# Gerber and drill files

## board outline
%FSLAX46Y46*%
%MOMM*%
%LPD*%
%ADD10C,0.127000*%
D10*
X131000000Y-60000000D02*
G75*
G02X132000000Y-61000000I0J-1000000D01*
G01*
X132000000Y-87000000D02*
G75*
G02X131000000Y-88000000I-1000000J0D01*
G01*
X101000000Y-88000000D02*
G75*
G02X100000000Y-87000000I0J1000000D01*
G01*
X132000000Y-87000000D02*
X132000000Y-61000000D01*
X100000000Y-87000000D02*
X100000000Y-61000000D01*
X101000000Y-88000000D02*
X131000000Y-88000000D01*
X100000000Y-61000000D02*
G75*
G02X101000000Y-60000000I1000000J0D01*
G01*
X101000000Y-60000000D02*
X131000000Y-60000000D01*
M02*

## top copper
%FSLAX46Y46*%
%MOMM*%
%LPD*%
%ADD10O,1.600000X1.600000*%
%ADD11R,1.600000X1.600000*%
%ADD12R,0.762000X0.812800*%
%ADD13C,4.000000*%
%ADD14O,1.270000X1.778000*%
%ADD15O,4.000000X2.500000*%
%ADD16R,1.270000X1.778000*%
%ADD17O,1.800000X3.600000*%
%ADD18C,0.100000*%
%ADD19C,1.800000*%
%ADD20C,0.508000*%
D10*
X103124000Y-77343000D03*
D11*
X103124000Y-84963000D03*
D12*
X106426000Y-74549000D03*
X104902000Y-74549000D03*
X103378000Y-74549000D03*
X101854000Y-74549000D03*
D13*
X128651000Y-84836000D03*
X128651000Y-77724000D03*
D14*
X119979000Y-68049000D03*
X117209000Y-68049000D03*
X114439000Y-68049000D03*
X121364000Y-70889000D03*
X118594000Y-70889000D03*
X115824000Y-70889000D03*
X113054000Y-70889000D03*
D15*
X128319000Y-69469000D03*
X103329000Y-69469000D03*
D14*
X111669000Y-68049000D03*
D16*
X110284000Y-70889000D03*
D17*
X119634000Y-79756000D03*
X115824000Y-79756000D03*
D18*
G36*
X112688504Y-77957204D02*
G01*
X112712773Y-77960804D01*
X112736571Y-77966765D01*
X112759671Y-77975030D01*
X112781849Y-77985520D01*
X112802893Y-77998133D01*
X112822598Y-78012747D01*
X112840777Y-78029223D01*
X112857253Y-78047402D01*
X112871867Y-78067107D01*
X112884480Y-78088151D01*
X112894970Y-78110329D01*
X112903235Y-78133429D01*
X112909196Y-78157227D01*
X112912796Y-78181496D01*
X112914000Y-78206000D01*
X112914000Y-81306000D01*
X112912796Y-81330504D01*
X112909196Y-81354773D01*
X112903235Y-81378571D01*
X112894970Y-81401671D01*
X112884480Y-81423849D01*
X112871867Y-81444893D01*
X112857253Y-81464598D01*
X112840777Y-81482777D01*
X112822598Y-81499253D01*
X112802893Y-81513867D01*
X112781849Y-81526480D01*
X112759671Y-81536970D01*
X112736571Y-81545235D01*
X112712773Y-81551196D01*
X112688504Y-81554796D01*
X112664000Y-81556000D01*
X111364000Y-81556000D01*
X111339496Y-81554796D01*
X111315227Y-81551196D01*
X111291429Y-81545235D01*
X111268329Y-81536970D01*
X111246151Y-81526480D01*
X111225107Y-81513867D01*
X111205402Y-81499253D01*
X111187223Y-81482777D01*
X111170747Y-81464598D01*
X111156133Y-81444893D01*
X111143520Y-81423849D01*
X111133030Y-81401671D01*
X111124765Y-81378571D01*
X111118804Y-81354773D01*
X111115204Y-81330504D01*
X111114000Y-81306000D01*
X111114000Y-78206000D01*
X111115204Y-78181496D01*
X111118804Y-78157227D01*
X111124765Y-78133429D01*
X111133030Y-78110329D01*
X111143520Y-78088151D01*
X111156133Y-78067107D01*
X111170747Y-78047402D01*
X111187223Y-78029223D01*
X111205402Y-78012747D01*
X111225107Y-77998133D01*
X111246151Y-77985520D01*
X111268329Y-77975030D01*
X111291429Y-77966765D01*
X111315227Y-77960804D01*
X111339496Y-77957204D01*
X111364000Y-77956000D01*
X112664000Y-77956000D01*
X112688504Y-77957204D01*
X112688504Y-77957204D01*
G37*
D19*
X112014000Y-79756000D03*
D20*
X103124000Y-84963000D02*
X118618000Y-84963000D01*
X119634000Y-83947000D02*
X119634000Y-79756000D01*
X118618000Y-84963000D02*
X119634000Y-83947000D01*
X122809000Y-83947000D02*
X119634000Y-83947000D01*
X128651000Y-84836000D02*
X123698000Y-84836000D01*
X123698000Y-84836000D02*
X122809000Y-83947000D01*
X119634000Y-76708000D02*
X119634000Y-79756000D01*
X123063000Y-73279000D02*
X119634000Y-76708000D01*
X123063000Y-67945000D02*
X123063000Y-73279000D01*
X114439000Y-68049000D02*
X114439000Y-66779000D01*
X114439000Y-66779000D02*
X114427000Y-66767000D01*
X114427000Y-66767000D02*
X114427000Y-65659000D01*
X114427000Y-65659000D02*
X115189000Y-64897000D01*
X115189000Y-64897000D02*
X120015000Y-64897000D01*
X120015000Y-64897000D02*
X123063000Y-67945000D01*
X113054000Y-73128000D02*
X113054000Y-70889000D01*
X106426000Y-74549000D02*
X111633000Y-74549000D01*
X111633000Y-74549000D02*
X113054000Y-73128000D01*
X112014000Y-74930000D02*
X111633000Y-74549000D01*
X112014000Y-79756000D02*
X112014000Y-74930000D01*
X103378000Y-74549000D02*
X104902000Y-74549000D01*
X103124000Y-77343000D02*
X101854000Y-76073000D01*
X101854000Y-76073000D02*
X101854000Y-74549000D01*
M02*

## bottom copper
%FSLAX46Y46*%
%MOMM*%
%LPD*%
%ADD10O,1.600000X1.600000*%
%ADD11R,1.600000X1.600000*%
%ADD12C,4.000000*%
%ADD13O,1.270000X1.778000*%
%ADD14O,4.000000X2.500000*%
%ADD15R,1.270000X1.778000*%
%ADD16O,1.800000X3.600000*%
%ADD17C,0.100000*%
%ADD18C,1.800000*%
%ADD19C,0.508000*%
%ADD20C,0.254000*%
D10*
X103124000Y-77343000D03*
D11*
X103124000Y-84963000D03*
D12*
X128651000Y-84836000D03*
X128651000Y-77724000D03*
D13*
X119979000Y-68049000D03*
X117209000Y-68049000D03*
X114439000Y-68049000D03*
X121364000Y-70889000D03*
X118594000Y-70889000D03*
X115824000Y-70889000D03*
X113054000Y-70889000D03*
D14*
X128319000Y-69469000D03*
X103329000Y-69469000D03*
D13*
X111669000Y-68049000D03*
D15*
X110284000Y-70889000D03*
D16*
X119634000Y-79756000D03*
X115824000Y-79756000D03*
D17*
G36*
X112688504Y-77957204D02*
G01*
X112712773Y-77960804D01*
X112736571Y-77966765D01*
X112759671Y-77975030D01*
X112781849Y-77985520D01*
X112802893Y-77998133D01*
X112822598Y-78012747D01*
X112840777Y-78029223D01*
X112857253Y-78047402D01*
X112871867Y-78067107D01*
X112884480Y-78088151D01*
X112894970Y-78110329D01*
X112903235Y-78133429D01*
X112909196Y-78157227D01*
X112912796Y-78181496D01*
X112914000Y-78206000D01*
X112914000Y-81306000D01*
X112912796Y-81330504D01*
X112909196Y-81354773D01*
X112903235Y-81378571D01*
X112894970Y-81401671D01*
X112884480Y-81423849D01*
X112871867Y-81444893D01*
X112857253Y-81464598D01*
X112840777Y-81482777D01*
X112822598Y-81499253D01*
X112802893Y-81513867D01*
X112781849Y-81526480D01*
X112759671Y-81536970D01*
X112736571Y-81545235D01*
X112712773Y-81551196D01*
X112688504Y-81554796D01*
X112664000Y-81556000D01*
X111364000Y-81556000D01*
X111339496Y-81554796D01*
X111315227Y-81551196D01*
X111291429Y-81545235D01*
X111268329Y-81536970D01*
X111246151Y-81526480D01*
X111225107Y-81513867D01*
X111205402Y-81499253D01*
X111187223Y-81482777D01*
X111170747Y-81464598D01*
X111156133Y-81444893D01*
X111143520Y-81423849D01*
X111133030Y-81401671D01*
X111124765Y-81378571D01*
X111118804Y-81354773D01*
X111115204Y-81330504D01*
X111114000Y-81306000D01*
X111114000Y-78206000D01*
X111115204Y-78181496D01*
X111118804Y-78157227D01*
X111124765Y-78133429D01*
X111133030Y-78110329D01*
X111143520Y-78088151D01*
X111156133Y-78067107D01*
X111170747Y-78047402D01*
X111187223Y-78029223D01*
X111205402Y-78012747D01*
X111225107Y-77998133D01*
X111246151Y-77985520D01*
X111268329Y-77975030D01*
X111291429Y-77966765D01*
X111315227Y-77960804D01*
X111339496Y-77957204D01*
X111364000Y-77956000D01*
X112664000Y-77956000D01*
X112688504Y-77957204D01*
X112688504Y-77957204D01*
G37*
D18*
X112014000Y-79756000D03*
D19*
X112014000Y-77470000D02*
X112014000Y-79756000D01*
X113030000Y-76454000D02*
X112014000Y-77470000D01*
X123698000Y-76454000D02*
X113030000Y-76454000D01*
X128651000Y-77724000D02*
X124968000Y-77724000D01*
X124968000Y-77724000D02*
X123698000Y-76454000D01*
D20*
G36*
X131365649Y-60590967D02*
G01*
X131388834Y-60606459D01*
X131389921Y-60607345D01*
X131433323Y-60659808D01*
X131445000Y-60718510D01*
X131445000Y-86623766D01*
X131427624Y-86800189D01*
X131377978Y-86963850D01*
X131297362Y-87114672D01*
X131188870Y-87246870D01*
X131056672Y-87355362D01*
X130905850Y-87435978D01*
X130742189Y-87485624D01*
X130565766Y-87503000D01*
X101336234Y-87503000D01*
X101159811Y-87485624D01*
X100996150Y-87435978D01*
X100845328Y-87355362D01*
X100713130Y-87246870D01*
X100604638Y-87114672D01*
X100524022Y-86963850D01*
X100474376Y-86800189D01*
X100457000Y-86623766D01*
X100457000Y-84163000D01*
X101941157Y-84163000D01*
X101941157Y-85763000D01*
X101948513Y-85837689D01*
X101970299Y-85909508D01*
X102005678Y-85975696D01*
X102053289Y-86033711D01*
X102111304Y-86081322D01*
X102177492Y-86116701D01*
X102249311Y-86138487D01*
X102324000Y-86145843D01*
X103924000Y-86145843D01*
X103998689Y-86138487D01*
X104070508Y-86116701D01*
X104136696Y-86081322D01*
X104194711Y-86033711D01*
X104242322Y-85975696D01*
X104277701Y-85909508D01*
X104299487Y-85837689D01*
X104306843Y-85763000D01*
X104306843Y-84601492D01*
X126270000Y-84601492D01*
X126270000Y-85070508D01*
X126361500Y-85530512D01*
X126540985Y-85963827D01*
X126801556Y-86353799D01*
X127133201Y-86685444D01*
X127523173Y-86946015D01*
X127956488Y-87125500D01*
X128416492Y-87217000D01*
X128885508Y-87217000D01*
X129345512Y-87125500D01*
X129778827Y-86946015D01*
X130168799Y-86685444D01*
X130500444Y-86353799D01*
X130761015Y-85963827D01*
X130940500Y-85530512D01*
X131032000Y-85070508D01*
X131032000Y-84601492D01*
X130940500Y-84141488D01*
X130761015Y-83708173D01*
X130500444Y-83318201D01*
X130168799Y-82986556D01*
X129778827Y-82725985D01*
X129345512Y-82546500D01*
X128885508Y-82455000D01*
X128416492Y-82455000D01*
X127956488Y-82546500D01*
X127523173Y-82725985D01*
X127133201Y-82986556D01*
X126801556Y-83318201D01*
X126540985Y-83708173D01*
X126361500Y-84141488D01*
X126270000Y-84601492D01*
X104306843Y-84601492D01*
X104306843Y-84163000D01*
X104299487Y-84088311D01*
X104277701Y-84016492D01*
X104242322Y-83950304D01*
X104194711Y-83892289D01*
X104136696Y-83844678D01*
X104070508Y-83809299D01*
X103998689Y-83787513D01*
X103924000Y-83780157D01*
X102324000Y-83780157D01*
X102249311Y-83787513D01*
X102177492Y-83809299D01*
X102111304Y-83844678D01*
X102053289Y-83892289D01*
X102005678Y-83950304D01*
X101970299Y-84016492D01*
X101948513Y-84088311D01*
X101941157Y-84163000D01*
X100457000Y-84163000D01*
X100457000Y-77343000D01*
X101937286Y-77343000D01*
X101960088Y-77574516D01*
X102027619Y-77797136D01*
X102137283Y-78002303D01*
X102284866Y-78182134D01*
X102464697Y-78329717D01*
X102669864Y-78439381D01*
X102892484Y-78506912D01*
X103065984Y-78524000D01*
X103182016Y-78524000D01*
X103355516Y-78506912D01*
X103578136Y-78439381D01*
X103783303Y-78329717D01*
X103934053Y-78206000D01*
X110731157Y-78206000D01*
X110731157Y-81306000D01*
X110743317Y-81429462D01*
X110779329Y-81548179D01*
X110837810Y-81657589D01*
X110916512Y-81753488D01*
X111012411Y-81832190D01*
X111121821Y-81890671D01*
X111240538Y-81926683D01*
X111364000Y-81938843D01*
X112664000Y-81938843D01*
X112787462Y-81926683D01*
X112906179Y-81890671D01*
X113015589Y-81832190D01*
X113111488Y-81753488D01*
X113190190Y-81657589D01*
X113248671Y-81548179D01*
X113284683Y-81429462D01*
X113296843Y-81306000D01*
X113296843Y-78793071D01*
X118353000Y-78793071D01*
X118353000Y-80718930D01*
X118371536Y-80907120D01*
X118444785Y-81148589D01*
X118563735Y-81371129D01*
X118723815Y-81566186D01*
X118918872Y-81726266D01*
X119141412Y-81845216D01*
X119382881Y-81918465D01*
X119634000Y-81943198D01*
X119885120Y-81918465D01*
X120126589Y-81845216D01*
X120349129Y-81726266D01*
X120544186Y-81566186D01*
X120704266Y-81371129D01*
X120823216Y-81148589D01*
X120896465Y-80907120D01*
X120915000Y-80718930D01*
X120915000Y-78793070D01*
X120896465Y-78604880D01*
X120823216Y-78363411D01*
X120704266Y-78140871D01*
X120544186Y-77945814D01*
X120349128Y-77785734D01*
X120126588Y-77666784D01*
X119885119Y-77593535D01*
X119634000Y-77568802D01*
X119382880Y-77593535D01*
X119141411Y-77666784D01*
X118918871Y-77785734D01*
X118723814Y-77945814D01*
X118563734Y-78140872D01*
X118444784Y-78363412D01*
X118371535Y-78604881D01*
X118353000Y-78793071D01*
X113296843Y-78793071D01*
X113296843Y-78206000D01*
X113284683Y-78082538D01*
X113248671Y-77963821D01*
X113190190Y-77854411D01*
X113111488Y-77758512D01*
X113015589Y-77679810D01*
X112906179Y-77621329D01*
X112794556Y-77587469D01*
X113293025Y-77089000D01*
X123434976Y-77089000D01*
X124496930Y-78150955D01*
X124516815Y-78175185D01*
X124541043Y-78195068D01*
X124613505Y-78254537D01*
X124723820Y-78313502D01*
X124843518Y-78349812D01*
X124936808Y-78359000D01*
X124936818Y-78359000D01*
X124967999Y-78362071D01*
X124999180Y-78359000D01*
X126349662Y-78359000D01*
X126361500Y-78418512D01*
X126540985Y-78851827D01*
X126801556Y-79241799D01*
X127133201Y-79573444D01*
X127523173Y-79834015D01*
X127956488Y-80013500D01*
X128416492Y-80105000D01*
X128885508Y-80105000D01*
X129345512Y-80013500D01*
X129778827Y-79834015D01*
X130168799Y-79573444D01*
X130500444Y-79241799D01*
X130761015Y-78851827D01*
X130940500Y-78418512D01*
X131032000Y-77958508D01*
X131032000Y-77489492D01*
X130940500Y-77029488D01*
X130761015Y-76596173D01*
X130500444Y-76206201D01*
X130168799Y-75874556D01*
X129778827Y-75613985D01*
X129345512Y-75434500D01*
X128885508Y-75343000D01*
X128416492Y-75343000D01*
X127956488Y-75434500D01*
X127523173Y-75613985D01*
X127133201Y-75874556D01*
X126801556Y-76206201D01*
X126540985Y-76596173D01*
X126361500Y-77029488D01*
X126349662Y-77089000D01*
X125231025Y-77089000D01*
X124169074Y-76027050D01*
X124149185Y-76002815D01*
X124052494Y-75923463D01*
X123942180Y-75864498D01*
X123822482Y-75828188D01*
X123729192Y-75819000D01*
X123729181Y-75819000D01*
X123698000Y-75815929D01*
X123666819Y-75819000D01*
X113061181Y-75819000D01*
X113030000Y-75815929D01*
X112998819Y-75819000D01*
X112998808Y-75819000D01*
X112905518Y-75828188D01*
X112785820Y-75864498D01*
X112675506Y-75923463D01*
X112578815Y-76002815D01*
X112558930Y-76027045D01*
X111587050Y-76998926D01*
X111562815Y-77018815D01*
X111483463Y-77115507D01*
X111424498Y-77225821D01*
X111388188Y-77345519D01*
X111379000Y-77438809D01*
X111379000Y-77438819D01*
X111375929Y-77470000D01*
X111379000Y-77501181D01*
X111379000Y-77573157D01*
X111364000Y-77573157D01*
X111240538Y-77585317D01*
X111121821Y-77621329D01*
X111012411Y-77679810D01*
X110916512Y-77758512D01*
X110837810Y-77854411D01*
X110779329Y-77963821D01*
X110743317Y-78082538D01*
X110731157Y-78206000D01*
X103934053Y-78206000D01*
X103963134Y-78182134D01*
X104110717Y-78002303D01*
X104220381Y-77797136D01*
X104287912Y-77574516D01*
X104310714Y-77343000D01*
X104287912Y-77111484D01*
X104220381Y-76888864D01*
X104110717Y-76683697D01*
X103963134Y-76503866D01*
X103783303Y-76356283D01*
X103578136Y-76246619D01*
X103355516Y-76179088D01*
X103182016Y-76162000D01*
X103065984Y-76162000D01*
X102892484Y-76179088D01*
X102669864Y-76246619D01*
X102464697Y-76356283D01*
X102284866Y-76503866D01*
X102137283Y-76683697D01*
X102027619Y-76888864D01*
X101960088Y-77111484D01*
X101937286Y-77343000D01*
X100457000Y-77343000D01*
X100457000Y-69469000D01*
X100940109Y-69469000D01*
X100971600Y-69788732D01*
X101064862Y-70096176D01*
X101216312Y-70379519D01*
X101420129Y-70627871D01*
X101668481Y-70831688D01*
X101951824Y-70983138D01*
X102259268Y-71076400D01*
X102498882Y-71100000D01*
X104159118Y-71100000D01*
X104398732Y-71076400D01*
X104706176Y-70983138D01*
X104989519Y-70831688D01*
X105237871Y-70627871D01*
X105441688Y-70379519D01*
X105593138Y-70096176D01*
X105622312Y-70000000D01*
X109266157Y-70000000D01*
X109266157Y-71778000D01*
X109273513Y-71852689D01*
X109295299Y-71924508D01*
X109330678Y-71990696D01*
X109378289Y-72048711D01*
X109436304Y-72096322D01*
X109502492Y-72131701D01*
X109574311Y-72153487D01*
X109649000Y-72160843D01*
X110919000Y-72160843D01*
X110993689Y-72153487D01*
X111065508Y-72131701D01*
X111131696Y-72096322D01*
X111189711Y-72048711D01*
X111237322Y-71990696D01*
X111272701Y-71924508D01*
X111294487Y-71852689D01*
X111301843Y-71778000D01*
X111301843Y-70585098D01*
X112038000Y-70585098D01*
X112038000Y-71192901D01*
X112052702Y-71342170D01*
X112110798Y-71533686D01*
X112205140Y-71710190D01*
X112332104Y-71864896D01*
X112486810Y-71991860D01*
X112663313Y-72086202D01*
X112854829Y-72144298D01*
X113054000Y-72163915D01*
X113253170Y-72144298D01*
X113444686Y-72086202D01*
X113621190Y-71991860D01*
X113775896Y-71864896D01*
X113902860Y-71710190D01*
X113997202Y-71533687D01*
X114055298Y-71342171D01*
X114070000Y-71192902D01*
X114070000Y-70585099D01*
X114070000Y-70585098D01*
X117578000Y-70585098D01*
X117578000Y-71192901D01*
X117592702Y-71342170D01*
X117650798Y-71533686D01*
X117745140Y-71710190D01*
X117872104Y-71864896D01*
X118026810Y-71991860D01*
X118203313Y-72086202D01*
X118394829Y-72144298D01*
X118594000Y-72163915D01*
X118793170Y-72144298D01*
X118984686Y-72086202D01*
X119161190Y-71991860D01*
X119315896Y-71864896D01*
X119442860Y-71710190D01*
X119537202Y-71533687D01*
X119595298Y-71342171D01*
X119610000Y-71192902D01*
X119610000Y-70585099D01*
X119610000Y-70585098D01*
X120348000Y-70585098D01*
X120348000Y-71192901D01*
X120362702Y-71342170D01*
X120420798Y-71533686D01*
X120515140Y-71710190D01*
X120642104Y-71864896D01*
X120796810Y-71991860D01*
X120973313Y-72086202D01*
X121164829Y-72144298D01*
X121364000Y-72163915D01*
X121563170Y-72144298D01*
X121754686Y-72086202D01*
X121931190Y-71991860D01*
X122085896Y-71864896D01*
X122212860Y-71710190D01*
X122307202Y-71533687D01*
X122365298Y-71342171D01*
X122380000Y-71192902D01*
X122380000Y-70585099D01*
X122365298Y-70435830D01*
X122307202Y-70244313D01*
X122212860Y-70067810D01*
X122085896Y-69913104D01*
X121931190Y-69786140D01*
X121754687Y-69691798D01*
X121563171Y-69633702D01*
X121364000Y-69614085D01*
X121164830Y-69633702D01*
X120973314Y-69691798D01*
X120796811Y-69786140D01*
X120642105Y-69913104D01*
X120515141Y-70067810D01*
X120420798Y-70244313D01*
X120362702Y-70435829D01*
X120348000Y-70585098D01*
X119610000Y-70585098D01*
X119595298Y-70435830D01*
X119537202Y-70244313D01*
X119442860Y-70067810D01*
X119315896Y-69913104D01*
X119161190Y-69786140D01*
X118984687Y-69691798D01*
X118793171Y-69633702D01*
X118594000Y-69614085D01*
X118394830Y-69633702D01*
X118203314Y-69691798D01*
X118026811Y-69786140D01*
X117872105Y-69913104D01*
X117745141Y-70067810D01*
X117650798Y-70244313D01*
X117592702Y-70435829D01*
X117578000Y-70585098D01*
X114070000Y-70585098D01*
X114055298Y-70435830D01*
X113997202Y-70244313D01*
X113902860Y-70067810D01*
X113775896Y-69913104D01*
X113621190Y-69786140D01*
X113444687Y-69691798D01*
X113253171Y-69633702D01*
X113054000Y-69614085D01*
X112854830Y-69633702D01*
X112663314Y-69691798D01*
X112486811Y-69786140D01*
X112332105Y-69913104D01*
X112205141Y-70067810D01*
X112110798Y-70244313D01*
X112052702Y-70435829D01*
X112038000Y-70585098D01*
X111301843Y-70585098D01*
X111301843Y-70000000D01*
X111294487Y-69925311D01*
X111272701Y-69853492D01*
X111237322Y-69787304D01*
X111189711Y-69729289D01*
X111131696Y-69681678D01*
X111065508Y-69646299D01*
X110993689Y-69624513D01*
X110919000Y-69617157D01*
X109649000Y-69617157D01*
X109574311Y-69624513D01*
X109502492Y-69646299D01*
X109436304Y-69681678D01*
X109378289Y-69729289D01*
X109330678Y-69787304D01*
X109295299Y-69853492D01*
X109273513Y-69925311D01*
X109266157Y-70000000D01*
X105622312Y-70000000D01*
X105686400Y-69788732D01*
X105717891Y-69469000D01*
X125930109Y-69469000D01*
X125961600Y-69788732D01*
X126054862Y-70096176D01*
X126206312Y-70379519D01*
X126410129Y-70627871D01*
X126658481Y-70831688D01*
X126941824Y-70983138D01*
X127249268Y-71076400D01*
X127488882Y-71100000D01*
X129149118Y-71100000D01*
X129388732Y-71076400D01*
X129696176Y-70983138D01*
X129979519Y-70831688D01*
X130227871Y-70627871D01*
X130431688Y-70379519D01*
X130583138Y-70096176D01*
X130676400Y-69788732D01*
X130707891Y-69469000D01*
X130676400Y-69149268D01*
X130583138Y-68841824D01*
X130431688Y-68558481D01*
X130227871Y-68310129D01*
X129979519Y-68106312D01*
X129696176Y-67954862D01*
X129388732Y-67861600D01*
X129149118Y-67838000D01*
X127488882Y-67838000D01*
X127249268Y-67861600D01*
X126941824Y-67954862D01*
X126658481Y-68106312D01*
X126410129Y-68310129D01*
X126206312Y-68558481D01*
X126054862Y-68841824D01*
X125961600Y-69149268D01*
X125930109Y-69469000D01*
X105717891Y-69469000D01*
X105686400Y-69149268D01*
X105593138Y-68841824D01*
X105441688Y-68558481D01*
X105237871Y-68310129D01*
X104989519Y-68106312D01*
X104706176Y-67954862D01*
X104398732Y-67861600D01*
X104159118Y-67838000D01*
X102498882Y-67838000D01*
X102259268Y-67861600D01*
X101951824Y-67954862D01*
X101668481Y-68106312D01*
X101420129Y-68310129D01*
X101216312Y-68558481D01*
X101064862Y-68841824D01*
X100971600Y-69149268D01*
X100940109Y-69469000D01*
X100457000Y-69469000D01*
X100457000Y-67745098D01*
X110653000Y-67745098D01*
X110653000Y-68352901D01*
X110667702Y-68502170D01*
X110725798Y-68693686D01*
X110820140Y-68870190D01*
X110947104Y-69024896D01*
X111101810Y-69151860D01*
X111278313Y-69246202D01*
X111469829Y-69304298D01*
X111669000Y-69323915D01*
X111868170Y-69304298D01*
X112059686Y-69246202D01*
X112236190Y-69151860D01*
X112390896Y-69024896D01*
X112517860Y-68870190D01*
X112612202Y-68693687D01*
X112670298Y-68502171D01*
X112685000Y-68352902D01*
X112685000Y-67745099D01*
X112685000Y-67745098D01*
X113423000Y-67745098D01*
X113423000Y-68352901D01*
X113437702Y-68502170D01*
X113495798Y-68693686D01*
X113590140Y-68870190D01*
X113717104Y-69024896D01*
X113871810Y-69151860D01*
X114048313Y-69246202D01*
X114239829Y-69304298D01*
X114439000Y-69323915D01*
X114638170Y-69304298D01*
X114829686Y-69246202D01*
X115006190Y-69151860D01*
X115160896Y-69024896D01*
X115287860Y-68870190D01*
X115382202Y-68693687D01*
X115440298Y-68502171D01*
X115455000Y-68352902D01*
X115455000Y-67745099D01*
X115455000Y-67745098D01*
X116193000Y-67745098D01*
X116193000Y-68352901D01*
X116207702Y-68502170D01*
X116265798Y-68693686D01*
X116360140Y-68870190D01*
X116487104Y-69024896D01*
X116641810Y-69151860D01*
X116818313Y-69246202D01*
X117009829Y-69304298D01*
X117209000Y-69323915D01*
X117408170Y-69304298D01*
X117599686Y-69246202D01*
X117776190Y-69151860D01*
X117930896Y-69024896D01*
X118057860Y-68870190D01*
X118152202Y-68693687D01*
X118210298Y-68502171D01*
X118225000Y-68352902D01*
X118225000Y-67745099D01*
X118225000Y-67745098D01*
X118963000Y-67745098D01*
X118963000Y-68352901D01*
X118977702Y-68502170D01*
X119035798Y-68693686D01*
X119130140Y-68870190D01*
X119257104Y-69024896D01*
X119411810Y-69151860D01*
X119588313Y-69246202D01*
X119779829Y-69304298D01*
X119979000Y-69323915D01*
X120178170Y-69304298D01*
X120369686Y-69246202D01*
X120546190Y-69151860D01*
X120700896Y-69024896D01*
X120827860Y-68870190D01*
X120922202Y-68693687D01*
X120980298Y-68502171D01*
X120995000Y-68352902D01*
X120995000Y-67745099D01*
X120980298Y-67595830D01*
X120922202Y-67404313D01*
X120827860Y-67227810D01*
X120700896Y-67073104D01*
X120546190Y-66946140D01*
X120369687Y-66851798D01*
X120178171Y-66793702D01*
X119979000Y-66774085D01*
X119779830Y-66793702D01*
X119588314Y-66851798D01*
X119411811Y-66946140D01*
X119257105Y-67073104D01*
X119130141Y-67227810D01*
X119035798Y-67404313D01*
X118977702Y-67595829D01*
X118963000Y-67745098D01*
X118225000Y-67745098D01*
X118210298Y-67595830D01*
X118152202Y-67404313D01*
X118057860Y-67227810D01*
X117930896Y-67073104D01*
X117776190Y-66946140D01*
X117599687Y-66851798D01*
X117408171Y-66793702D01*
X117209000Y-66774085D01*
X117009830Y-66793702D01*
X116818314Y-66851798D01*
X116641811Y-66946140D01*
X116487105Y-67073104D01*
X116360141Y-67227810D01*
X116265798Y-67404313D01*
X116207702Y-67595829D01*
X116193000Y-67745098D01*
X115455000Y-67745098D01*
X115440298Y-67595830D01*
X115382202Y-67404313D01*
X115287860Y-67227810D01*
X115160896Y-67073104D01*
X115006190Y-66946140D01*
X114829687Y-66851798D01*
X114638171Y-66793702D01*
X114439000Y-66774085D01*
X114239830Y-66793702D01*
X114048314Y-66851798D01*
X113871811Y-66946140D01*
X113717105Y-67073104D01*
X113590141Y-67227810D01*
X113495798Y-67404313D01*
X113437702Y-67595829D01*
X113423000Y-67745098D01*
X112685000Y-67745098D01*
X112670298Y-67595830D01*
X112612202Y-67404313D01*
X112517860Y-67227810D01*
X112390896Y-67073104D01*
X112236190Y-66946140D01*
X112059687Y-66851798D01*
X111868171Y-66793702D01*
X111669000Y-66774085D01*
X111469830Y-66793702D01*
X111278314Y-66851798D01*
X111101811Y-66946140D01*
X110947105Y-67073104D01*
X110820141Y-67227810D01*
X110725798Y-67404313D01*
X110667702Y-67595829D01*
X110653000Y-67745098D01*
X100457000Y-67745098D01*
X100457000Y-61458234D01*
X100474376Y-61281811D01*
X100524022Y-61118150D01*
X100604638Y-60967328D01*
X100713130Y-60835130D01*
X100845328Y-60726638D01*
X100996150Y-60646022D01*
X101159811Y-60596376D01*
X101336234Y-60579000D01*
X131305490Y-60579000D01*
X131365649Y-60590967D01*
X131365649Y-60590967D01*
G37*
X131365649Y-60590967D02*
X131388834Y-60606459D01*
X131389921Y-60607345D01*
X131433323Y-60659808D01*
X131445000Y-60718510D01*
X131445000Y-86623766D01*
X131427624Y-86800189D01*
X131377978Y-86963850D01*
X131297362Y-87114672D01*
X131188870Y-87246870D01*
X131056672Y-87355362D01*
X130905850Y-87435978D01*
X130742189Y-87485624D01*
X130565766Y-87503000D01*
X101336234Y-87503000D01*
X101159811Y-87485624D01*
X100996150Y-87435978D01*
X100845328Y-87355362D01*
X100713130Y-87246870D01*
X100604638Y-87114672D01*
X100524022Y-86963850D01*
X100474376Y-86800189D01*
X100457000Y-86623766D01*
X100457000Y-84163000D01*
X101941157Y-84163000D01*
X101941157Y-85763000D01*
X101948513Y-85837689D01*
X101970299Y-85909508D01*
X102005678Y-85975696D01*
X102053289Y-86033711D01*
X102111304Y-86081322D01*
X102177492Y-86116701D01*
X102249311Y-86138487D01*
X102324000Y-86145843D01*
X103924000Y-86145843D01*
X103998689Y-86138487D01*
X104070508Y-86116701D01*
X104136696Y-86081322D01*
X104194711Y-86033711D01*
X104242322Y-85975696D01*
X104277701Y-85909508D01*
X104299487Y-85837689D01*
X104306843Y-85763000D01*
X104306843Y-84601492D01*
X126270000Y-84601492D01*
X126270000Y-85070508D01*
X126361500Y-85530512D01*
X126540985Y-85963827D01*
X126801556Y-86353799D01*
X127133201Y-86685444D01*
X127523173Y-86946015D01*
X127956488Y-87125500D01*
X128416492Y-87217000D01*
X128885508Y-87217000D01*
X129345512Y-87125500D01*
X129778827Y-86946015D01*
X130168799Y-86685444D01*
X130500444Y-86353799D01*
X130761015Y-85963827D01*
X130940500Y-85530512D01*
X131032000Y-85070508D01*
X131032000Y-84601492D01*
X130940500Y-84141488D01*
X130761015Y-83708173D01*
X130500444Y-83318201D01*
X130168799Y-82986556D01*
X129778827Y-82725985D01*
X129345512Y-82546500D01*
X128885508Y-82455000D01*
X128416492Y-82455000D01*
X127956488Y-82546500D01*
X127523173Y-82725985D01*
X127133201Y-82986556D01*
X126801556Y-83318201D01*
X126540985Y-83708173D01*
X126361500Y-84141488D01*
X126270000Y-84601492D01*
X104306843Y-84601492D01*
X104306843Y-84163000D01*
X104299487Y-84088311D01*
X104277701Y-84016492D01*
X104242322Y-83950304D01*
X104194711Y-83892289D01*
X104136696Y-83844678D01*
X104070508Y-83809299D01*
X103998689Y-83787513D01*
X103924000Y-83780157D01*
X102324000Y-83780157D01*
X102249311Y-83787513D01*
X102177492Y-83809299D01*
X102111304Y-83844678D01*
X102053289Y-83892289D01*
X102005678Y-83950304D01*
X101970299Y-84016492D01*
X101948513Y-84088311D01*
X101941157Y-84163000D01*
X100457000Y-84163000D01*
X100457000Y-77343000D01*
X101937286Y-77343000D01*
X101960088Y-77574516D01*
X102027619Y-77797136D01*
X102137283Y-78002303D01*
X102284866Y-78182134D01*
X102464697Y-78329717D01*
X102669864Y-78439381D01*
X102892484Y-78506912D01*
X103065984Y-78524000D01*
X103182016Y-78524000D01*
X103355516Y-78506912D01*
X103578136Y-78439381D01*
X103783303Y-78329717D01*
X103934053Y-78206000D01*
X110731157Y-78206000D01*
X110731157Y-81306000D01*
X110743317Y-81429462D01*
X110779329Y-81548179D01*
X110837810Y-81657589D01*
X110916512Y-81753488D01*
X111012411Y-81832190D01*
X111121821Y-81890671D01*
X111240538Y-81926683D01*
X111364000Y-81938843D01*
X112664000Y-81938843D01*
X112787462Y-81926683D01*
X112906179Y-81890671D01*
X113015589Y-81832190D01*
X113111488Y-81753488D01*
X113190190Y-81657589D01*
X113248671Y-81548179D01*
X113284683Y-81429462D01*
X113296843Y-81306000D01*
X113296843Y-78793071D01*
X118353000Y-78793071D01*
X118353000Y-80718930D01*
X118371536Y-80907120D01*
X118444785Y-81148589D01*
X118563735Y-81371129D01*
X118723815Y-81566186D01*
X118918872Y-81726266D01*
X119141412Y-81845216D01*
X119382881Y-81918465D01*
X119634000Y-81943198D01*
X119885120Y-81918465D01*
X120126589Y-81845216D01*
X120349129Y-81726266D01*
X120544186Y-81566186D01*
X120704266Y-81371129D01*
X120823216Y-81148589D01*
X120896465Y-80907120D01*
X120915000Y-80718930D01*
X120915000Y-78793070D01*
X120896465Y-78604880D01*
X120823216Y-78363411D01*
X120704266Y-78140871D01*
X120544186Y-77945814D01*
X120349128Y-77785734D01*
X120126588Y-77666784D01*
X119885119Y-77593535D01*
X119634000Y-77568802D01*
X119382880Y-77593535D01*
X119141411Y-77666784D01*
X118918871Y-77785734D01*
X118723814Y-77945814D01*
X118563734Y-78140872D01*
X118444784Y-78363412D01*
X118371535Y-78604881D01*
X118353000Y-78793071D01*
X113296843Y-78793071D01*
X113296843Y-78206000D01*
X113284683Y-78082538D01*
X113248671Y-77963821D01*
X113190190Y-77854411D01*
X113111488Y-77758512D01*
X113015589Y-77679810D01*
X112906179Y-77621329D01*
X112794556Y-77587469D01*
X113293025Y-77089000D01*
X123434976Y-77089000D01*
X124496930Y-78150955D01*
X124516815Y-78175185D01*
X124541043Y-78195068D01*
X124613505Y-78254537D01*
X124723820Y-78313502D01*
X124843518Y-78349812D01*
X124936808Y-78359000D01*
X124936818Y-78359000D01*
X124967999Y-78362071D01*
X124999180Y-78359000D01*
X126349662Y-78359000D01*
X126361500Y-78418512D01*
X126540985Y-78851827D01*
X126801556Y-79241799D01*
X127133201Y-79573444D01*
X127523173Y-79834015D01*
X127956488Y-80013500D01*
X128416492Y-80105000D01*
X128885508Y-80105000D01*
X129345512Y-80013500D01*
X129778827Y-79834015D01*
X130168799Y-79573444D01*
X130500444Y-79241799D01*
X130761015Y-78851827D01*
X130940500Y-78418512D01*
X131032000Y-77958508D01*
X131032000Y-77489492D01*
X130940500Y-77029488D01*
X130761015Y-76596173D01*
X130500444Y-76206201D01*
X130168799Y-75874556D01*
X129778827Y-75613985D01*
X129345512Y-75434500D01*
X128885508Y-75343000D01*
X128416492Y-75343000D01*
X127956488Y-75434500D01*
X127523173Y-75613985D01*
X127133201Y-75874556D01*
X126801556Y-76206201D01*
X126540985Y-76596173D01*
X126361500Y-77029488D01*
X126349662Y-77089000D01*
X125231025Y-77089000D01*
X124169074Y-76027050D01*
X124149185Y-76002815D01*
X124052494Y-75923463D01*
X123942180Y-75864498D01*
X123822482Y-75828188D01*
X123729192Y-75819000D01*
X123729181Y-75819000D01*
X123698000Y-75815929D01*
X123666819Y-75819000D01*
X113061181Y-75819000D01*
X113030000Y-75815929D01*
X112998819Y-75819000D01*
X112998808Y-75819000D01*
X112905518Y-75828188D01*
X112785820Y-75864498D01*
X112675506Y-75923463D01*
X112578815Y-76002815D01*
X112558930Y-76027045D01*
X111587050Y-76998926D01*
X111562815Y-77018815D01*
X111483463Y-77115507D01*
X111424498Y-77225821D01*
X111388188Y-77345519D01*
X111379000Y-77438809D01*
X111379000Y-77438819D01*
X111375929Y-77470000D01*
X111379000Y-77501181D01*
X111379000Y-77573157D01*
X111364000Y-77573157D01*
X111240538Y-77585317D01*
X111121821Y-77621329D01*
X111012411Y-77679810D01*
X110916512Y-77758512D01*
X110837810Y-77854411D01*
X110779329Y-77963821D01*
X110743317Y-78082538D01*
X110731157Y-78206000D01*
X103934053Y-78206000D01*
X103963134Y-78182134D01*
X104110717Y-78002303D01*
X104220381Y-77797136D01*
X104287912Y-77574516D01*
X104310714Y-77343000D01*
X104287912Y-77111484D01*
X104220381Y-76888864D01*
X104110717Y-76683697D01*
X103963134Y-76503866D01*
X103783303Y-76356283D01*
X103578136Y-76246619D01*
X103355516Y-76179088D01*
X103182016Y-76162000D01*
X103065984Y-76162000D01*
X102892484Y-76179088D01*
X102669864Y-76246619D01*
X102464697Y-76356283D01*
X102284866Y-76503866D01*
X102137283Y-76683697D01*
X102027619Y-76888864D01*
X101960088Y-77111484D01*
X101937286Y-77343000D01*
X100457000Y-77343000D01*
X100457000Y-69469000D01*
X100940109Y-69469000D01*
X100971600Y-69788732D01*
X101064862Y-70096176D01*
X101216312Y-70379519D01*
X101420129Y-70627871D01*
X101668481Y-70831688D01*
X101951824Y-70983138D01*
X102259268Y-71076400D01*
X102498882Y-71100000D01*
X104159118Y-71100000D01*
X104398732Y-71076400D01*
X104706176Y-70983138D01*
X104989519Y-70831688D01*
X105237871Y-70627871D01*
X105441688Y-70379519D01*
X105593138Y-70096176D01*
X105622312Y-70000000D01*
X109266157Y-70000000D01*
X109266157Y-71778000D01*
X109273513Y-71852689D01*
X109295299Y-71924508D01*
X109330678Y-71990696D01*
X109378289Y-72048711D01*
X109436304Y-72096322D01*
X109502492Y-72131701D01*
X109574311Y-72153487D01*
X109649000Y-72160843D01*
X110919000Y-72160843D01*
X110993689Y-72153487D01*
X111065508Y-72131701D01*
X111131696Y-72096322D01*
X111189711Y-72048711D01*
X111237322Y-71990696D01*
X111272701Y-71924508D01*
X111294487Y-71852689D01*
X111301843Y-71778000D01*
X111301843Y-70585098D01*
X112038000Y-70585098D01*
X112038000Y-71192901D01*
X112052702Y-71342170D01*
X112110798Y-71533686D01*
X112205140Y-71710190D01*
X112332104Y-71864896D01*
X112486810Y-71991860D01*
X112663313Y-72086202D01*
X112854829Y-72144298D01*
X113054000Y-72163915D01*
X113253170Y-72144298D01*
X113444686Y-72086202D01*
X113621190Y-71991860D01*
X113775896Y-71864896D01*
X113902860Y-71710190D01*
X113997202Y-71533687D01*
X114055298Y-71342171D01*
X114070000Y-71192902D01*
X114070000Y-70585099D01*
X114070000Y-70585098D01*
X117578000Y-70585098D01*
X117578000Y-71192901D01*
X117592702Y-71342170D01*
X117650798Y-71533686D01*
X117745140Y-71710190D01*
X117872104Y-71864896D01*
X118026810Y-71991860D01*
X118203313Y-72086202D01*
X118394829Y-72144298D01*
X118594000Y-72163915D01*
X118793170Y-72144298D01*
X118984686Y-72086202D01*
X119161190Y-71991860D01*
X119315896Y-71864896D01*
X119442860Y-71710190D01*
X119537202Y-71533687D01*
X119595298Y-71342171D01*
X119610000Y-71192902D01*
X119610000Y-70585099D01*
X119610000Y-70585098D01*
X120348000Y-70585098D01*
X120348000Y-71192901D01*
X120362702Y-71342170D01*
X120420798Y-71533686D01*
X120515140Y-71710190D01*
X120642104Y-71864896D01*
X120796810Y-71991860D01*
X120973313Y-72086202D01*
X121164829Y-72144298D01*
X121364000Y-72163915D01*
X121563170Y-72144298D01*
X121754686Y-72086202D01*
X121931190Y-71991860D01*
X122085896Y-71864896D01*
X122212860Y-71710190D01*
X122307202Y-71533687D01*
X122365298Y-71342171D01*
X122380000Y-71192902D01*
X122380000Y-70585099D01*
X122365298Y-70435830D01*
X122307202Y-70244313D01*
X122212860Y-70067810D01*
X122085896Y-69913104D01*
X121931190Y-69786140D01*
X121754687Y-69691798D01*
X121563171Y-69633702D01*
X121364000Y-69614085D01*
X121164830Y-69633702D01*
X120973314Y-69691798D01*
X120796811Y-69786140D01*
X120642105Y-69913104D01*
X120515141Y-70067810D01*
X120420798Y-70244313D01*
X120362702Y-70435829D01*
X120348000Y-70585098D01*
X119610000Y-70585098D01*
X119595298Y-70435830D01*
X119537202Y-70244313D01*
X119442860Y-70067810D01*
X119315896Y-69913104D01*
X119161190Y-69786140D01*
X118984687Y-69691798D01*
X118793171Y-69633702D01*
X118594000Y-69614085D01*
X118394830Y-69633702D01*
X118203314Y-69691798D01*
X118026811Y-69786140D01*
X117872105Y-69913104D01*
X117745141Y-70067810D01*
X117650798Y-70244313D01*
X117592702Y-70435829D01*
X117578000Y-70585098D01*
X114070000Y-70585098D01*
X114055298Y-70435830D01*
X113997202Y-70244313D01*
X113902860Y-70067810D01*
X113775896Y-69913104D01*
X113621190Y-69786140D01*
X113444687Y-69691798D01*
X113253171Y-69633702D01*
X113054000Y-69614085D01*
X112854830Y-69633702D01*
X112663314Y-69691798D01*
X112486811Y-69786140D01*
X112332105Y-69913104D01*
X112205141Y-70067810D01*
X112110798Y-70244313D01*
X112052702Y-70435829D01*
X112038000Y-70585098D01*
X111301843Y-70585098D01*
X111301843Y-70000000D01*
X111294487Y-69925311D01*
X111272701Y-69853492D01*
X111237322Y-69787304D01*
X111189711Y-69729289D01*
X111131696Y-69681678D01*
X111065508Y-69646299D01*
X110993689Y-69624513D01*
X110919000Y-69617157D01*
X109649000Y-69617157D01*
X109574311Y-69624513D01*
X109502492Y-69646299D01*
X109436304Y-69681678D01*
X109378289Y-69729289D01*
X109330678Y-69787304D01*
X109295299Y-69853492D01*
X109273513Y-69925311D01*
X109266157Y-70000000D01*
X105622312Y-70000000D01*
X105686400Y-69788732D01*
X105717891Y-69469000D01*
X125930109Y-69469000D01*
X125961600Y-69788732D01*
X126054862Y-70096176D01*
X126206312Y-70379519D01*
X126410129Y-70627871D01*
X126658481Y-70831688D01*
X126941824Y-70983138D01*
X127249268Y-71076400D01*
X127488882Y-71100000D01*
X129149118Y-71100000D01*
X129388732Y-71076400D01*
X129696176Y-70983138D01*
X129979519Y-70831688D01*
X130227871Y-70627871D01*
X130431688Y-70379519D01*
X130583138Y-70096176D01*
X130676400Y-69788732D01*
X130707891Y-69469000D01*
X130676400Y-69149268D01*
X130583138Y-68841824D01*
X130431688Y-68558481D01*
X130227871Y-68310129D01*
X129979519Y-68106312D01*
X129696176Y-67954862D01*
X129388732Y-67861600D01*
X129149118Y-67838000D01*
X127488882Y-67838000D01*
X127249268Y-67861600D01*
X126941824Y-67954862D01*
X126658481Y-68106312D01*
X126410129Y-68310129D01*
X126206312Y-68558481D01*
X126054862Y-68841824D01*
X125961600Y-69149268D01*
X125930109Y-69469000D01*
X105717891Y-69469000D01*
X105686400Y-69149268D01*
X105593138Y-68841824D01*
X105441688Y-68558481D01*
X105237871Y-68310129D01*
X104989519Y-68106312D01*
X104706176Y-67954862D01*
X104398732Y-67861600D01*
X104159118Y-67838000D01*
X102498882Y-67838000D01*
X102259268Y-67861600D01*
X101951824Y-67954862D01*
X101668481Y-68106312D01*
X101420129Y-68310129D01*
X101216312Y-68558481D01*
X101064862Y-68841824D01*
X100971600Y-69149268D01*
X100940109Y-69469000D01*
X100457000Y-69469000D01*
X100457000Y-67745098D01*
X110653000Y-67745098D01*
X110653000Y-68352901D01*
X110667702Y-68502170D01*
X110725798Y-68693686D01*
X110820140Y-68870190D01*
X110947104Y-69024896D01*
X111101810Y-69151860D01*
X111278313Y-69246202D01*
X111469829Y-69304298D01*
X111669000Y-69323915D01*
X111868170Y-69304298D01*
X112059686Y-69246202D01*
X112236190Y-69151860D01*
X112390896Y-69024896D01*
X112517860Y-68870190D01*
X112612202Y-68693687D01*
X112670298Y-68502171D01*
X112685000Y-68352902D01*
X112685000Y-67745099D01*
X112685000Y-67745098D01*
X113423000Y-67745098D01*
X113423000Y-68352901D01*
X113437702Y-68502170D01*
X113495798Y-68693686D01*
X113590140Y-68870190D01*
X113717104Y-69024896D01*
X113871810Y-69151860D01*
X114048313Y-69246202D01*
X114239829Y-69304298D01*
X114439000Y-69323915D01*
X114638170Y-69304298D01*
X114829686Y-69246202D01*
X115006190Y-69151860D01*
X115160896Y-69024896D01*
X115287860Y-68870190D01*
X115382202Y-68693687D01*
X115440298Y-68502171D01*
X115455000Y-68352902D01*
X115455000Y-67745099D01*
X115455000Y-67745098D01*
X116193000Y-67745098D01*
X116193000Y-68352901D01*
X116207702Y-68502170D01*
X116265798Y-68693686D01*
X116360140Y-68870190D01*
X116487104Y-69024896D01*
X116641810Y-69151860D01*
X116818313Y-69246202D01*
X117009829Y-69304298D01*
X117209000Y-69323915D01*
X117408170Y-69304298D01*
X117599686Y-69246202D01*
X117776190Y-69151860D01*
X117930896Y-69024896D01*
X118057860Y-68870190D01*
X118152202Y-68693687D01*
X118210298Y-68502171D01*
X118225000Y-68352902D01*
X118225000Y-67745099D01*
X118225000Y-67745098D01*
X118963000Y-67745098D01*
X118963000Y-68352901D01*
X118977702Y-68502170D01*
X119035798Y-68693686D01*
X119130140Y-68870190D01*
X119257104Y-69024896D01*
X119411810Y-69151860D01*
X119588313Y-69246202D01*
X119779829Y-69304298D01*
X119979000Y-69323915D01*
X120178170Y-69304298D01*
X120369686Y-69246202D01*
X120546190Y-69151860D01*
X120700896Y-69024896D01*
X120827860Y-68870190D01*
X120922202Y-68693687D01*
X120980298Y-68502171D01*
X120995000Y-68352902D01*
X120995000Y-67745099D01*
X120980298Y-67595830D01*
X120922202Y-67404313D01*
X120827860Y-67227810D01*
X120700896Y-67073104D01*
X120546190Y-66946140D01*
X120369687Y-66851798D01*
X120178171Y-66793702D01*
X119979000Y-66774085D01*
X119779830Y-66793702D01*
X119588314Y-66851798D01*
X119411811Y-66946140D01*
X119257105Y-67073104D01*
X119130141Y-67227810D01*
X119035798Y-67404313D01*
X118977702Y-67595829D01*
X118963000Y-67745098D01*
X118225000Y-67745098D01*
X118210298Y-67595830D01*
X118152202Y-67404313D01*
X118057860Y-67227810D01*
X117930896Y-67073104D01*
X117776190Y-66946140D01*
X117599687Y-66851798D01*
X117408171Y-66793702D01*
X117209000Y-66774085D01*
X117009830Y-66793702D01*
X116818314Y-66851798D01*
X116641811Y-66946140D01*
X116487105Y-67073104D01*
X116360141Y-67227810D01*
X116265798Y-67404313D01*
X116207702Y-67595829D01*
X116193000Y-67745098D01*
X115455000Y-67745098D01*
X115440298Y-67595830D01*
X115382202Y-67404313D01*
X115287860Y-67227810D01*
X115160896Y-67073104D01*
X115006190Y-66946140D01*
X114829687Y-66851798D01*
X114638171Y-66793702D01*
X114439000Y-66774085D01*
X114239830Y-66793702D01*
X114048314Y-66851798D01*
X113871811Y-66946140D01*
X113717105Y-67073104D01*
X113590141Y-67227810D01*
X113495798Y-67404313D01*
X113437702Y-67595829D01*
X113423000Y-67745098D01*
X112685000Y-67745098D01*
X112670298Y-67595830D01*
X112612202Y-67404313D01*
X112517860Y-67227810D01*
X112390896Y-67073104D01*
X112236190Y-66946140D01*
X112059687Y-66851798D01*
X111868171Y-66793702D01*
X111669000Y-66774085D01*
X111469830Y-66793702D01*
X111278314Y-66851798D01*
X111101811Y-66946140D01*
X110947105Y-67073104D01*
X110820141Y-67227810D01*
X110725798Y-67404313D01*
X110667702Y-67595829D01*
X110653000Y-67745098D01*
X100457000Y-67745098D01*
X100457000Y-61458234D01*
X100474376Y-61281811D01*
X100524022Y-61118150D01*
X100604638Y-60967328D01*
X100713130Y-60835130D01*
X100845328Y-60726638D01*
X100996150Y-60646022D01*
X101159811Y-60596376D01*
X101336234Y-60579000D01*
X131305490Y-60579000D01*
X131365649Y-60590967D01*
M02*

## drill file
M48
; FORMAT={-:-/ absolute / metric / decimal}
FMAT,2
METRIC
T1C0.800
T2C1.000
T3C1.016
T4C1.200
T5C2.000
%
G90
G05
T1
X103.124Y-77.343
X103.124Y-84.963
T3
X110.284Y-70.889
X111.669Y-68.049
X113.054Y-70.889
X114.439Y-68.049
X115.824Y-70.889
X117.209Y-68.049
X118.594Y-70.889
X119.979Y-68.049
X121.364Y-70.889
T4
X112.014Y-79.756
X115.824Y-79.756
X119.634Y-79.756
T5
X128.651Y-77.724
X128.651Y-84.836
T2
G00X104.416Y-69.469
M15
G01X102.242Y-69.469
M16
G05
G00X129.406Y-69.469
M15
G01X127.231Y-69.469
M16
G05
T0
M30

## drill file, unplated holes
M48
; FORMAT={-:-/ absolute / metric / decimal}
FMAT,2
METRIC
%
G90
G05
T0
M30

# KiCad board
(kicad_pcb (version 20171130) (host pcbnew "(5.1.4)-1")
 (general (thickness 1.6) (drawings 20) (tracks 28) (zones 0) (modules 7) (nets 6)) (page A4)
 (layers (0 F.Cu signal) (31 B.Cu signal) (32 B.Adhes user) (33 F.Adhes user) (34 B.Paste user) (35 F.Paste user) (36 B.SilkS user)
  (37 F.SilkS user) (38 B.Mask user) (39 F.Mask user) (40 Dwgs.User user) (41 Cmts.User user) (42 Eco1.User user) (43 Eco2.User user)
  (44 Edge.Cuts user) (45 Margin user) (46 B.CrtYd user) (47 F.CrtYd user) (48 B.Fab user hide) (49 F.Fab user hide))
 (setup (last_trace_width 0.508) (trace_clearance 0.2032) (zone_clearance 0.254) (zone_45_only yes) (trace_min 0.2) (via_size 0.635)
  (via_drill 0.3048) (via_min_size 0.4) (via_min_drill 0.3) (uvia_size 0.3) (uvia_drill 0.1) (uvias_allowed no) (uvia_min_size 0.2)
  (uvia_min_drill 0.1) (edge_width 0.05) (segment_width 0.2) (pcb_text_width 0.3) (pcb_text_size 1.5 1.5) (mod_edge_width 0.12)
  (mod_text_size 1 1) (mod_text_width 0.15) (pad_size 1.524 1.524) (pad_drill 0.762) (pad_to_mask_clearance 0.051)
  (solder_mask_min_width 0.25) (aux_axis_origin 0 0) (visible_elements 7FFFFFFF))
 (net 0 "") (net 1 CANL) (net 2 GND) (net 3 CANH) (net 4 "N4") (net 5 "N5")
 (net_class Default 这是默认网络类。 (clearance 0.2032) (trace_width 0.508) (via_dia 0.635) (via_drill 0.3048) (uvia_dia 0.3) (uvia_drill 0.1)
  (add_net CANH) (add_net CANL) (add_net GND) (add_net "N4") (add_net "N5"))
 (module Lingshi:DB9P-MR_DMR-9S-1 (layer F.Cu) (at 115.824 69.469 180)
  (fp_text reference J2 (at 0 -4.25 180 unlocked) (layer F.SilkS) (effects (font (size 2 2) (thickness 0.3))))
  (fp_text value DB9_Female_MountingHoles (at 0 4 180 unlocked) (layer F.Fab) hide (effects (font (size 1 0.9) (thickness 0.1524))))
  (pad 1 thru_hole rect (at 5.54 -1.42 270) (size 1.778 1.27) (drill 1.016) (layers *.Cu *.Mask))
  (pad 6 thru_hole oval (at 4.155 1.42 270) (size 1.778 1.27) (drill 1.016) (layers *.Cu *.Mask))
  (pad 10 thru_hole oval (at 12.495 0 180) (size 4 2.5) (drill oval 3.175 1) (layers *.Cu *.Mask))
  (pad 11 thru_hole oval (at -12.495 0 180) (size 4 2.5) (drill oval 3.175 1) (layers *.Cu *.Mask))
  (pad 2 thru_hole oval (at 2.77 -1.42 270) (size 1.778 1.27) (drill 1.016) (layers *.Cu *.Mask) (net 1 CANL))
  (pad 3 thru_hole oval (at 0 -1.42 270) (size 1.778 1.27) (drill 1.016) (layers *.Cu *.Mask) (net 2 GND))
  (pad 4 thru_hole oval (at -2.77 -1.42 270) (size 1.778 1.27) (drill 1.016) (layers *.Cu *.Mask))
  (pad 5 thru_hole oval (at -5.54 -1.42 270) (size 1.778 1.27) (drill 1.016) (layers *.Cu *.Mask))
  (pad 7 thru_hole oval (at 1.385 1.42 270) (size 1.778 1.27) (drill 1.016) (layers *.Cu *.Mask) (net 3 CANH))
  (pad 8 thru_hole oval (at -1.385 1.42 270) (size 1.778 1.27) (drill 1.016) (layers *.Cu *.Mask))
  (pad 9 thru_hole oval (at -4.155 1.42 270) (size 1.778 1.27) (drill 1.016) (layers *.Cu *.Mask)))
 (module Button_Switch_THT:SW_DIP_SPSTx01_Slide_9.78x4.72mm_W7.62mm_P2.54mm (layer F.Cu) (at 103.124 84.963 90)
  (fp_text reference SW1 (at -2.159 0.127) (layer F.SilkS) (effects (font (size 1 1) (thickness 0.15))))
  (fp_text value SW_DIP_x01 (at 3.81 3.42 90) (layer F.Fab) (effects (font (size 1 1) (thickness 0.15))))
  (pad 2 thru_hole oval (at 7.62 0 90) (size 1.6 1.6) (drill 0.8) (layers *.Cu *.Mask) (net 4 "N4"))
  (pad 1 thru_hole rect (at 0 0 90) (size 1.6 1.6) (drill 0.8) (layers *.Cu *.Mask) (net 3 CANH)))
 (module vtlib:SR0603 (layer F.Cu) (at 105.664 74.549)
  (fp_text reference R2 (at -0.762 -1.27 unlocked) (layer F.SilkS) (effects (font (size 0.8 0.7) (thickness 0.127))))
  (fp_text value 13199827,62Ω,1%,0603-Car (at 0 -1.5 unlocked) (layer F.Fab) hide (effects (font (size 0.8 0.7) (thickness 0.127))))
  (pad 2 smd rect (at 0.762 0 90) (size 0.8128 0.762) (layers F.Cu F.Paste F.Mask) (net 1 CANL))
  (pad 1 smd rect (at -0.762 0 90) (size 0.8128 0.762) (layers F.Cu F.Paste F.Mask) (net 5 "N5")))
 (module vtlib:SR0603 (layer F.Cu) (at 102.616 74.549)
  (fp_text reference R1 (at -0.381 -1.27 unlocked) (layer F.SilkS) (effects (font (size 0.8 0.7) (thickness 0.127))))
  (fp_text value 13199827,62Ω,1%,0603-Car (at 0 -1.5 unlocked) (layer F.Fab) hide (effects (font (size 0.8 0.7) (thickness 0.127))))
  (pad 2 smd rect (at 0.762 0 90) (size 0.8128 0.762) (layers F.Cu F.Paste F.Mask) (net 5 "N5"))
  (pad 1 smd rect (at -0.762 0 90) (size 0.8128 0.762) (layers F.Cu F.Paste F.Mask) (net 4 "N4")))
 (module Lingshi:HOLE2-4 (layer F.Cu) (at 128.651 84.836)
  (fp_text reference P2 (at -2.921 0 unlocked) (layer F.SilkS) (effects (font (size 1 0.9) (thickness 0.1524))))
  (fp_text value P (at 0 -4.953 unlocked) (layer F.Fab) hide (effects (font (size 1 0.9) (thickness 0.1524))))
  (pad 1 thru_hole circle (at 0 0) (size 4 4) (drill 2) (layers *.Cu *.Mask) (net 3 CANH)))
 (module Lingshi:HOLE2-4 (layer F.Cu) (at 128.651 77.724)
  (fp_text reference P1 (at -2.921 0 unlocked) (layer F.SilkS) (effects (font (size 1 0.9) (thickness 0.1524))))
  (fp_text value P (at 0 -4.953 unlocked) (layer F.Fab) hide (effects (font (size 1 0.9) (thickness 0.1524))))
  (pad 1 thru_hole circle (at 0 0) (size 4 4) (drill 2) (layers *.Cu *.Mask) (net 1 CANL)))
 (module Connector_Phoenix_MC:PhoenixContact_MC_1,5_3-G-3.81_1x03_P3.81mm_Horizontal (layer F.Cu) (at 112.014 79.756)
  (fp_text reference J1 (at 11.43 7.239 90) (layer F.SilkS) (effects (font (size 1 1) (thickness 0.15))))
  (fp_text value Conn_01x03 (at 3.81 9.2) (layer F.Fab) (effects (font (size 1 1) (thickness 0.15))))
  (pad 3 thru_hole oval (at 7.62 0) (size 1.8 3.6) (drill 1.2) (layers *.Cu *.Mask) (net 3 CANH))
  (pad 2 thru_hole oval (at 3.81 0) (size 1.8 3.6) (drill 1.2) (layers *.Cu *.Mask) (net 2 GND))
  (pad 1 thru_hole roundrect (at 0 0) (size 1.8 3.6) (drill 1.2) (layers *.Cu *.Mask) (roundrect_rratio 0.138889) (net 1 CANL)))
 (gr_arc (start 131 61) (end 132 61) (angle -90) (layer Edge.Cuts) (width 0.127))
 (gr_arc (start 131 87) (end 131 88) (angle -90) (layer Edge.Cuts) (width 0.127))
 (gr_arc (start 101 87) (end 100 87) (angle -90) (layer Edge.Cuts) (width 0.127))
 (gr_line (start 132 87) (end 132 61) (layer Edge.Cuts) (width 0.127))
 (gr_line (start 100 87) (end 100 61) (layer Edge.Cuts) (width 0.127))
 (gr_line (start 101 88) (end 131 88) (layer Edge.Cuts) (width 0.127))
 (gr_arc (start 101 61) (end 101 60) (angle -90) (layer Edge.Cuts) (width 0.127))
 (gr_line (start 101 60) (end 131 60) (layer Edge.Cuts) (width 0.127))
 (segment (start 103.124 84.963) (end 118.618 84.963) (width 0.508) (layer F.Cu) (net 3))
 (segment (start 119.634 83.947) (end 119.634 79.756) (width 0.508) (layer F.Cu) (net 3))
 (segment (start 118.618 84.963) (end 119.634 83.947) (width 0.508) (layer F.Cu) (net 3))
 (segment (start 122.809 83.947) (end 119.634 83.947) (width 0.508) (layer F.Cu) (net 3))
 (segment (start 128.651 84.836) (end 123.698 84.836) (width 0.508) (layer F.Cu) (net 3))
 (segment (start 123.698 84.836) (end 122.809 83.947) (width 0.508) (layer F.Cu) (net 3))
 (segment (start 119.634 76.708) (end 119.634 79.756) (width 0.508) (layer F.Cu) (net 3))
 (segment (start 123.063 73.279) (end 119.634 76.708) (width 0.508) (layer F.Cu) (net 3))
 (segment (start 123.063 67.945) (end 123.063 73.279) (width 0.508) (layer F.Cu) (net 3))
 (segment (start 114.439 68.049) (end 114.439 66.779) (width 0.508) (layer F.Cu) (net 3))
 (segment (start 114.439 66.779) (end 114.427 66.767) (width 0.508) (layer F.Cu) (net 3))
 (segment (start 114.427 66.767) (end 114.427 65.659) (width 0.508) (layer F.Cu) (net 3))
 (segment (start 114.427 65.659) (end 115.189 64.897) (width 0.508) (layer F.Cu) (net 3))
 (segment (start 115.189 64.897) (end 120.015 64.897) (width 0.508) (layer F.Cu) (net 3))
 (segment (start 120.015 64.897) (end 123.063 67.945) (width 0.508) (layer F.Cu) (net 3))
 (segment (start 113.054 73.128) (end 113.054 70.889) (width 0.508) (layer F.Cu) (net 1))
 (segment (start 106.426 74.549) (end 111.633 74.549) (width 0.508) (layer F.Cu) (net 1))
 (segment (start 111.633 74.549) (end 113.054 73.128) (width 0.508) (layer F.Cu) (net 1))
 (segment (start 112.014 74.93) (end 111.633 74.549) (width 0.508) (layer F.Cu) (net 1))
 (segment (start 112.014 79.756) (end 112.014 74.93) (width 0.508) (layer F.Cu) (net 1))
 (segment (start 112.014 77.47) (end 112.014 79.756) (width 0.508) (layer B.Cu) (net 1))
 (segment (start 113.03 76.454) (end 112.014 77.47) (width 0.508) (layer B.Cu) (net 1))
 (segment (start 123.698 76.454) (end 113.03 76.454) (width 0.508) (layer B.Cu) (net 1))
 (segment (start 128.651 77.724) (end 124.968 77.724) (width 0.508) (layer B.Cu) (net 1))
 (segment (start 124.968 77.724) (end 123.698 76.454) (width 0.508) (layer B.Cu) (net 1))
 (segment (start 103.378 74.549) (end 104.902 74.549) (width 0.508) (layer F.Cu) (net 5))
 (segment (start 103.124 77.343) (end 101.854 76.073) (width 0.508) (layer F.Cu) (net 4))
 (segment (start 101.854 76.073) (end 101.854 74.549) (width 0.508) (layer F.Cu) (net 4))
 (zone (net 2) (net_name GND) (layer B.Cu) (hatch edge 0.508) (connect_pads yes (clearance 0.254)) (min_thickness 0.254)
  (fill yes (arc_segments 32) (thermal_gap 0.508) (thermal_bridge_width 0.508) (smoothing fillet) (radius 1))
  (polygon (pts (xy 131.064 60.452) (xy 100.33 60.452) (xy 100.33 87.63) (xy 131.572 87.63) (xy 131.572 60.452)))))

